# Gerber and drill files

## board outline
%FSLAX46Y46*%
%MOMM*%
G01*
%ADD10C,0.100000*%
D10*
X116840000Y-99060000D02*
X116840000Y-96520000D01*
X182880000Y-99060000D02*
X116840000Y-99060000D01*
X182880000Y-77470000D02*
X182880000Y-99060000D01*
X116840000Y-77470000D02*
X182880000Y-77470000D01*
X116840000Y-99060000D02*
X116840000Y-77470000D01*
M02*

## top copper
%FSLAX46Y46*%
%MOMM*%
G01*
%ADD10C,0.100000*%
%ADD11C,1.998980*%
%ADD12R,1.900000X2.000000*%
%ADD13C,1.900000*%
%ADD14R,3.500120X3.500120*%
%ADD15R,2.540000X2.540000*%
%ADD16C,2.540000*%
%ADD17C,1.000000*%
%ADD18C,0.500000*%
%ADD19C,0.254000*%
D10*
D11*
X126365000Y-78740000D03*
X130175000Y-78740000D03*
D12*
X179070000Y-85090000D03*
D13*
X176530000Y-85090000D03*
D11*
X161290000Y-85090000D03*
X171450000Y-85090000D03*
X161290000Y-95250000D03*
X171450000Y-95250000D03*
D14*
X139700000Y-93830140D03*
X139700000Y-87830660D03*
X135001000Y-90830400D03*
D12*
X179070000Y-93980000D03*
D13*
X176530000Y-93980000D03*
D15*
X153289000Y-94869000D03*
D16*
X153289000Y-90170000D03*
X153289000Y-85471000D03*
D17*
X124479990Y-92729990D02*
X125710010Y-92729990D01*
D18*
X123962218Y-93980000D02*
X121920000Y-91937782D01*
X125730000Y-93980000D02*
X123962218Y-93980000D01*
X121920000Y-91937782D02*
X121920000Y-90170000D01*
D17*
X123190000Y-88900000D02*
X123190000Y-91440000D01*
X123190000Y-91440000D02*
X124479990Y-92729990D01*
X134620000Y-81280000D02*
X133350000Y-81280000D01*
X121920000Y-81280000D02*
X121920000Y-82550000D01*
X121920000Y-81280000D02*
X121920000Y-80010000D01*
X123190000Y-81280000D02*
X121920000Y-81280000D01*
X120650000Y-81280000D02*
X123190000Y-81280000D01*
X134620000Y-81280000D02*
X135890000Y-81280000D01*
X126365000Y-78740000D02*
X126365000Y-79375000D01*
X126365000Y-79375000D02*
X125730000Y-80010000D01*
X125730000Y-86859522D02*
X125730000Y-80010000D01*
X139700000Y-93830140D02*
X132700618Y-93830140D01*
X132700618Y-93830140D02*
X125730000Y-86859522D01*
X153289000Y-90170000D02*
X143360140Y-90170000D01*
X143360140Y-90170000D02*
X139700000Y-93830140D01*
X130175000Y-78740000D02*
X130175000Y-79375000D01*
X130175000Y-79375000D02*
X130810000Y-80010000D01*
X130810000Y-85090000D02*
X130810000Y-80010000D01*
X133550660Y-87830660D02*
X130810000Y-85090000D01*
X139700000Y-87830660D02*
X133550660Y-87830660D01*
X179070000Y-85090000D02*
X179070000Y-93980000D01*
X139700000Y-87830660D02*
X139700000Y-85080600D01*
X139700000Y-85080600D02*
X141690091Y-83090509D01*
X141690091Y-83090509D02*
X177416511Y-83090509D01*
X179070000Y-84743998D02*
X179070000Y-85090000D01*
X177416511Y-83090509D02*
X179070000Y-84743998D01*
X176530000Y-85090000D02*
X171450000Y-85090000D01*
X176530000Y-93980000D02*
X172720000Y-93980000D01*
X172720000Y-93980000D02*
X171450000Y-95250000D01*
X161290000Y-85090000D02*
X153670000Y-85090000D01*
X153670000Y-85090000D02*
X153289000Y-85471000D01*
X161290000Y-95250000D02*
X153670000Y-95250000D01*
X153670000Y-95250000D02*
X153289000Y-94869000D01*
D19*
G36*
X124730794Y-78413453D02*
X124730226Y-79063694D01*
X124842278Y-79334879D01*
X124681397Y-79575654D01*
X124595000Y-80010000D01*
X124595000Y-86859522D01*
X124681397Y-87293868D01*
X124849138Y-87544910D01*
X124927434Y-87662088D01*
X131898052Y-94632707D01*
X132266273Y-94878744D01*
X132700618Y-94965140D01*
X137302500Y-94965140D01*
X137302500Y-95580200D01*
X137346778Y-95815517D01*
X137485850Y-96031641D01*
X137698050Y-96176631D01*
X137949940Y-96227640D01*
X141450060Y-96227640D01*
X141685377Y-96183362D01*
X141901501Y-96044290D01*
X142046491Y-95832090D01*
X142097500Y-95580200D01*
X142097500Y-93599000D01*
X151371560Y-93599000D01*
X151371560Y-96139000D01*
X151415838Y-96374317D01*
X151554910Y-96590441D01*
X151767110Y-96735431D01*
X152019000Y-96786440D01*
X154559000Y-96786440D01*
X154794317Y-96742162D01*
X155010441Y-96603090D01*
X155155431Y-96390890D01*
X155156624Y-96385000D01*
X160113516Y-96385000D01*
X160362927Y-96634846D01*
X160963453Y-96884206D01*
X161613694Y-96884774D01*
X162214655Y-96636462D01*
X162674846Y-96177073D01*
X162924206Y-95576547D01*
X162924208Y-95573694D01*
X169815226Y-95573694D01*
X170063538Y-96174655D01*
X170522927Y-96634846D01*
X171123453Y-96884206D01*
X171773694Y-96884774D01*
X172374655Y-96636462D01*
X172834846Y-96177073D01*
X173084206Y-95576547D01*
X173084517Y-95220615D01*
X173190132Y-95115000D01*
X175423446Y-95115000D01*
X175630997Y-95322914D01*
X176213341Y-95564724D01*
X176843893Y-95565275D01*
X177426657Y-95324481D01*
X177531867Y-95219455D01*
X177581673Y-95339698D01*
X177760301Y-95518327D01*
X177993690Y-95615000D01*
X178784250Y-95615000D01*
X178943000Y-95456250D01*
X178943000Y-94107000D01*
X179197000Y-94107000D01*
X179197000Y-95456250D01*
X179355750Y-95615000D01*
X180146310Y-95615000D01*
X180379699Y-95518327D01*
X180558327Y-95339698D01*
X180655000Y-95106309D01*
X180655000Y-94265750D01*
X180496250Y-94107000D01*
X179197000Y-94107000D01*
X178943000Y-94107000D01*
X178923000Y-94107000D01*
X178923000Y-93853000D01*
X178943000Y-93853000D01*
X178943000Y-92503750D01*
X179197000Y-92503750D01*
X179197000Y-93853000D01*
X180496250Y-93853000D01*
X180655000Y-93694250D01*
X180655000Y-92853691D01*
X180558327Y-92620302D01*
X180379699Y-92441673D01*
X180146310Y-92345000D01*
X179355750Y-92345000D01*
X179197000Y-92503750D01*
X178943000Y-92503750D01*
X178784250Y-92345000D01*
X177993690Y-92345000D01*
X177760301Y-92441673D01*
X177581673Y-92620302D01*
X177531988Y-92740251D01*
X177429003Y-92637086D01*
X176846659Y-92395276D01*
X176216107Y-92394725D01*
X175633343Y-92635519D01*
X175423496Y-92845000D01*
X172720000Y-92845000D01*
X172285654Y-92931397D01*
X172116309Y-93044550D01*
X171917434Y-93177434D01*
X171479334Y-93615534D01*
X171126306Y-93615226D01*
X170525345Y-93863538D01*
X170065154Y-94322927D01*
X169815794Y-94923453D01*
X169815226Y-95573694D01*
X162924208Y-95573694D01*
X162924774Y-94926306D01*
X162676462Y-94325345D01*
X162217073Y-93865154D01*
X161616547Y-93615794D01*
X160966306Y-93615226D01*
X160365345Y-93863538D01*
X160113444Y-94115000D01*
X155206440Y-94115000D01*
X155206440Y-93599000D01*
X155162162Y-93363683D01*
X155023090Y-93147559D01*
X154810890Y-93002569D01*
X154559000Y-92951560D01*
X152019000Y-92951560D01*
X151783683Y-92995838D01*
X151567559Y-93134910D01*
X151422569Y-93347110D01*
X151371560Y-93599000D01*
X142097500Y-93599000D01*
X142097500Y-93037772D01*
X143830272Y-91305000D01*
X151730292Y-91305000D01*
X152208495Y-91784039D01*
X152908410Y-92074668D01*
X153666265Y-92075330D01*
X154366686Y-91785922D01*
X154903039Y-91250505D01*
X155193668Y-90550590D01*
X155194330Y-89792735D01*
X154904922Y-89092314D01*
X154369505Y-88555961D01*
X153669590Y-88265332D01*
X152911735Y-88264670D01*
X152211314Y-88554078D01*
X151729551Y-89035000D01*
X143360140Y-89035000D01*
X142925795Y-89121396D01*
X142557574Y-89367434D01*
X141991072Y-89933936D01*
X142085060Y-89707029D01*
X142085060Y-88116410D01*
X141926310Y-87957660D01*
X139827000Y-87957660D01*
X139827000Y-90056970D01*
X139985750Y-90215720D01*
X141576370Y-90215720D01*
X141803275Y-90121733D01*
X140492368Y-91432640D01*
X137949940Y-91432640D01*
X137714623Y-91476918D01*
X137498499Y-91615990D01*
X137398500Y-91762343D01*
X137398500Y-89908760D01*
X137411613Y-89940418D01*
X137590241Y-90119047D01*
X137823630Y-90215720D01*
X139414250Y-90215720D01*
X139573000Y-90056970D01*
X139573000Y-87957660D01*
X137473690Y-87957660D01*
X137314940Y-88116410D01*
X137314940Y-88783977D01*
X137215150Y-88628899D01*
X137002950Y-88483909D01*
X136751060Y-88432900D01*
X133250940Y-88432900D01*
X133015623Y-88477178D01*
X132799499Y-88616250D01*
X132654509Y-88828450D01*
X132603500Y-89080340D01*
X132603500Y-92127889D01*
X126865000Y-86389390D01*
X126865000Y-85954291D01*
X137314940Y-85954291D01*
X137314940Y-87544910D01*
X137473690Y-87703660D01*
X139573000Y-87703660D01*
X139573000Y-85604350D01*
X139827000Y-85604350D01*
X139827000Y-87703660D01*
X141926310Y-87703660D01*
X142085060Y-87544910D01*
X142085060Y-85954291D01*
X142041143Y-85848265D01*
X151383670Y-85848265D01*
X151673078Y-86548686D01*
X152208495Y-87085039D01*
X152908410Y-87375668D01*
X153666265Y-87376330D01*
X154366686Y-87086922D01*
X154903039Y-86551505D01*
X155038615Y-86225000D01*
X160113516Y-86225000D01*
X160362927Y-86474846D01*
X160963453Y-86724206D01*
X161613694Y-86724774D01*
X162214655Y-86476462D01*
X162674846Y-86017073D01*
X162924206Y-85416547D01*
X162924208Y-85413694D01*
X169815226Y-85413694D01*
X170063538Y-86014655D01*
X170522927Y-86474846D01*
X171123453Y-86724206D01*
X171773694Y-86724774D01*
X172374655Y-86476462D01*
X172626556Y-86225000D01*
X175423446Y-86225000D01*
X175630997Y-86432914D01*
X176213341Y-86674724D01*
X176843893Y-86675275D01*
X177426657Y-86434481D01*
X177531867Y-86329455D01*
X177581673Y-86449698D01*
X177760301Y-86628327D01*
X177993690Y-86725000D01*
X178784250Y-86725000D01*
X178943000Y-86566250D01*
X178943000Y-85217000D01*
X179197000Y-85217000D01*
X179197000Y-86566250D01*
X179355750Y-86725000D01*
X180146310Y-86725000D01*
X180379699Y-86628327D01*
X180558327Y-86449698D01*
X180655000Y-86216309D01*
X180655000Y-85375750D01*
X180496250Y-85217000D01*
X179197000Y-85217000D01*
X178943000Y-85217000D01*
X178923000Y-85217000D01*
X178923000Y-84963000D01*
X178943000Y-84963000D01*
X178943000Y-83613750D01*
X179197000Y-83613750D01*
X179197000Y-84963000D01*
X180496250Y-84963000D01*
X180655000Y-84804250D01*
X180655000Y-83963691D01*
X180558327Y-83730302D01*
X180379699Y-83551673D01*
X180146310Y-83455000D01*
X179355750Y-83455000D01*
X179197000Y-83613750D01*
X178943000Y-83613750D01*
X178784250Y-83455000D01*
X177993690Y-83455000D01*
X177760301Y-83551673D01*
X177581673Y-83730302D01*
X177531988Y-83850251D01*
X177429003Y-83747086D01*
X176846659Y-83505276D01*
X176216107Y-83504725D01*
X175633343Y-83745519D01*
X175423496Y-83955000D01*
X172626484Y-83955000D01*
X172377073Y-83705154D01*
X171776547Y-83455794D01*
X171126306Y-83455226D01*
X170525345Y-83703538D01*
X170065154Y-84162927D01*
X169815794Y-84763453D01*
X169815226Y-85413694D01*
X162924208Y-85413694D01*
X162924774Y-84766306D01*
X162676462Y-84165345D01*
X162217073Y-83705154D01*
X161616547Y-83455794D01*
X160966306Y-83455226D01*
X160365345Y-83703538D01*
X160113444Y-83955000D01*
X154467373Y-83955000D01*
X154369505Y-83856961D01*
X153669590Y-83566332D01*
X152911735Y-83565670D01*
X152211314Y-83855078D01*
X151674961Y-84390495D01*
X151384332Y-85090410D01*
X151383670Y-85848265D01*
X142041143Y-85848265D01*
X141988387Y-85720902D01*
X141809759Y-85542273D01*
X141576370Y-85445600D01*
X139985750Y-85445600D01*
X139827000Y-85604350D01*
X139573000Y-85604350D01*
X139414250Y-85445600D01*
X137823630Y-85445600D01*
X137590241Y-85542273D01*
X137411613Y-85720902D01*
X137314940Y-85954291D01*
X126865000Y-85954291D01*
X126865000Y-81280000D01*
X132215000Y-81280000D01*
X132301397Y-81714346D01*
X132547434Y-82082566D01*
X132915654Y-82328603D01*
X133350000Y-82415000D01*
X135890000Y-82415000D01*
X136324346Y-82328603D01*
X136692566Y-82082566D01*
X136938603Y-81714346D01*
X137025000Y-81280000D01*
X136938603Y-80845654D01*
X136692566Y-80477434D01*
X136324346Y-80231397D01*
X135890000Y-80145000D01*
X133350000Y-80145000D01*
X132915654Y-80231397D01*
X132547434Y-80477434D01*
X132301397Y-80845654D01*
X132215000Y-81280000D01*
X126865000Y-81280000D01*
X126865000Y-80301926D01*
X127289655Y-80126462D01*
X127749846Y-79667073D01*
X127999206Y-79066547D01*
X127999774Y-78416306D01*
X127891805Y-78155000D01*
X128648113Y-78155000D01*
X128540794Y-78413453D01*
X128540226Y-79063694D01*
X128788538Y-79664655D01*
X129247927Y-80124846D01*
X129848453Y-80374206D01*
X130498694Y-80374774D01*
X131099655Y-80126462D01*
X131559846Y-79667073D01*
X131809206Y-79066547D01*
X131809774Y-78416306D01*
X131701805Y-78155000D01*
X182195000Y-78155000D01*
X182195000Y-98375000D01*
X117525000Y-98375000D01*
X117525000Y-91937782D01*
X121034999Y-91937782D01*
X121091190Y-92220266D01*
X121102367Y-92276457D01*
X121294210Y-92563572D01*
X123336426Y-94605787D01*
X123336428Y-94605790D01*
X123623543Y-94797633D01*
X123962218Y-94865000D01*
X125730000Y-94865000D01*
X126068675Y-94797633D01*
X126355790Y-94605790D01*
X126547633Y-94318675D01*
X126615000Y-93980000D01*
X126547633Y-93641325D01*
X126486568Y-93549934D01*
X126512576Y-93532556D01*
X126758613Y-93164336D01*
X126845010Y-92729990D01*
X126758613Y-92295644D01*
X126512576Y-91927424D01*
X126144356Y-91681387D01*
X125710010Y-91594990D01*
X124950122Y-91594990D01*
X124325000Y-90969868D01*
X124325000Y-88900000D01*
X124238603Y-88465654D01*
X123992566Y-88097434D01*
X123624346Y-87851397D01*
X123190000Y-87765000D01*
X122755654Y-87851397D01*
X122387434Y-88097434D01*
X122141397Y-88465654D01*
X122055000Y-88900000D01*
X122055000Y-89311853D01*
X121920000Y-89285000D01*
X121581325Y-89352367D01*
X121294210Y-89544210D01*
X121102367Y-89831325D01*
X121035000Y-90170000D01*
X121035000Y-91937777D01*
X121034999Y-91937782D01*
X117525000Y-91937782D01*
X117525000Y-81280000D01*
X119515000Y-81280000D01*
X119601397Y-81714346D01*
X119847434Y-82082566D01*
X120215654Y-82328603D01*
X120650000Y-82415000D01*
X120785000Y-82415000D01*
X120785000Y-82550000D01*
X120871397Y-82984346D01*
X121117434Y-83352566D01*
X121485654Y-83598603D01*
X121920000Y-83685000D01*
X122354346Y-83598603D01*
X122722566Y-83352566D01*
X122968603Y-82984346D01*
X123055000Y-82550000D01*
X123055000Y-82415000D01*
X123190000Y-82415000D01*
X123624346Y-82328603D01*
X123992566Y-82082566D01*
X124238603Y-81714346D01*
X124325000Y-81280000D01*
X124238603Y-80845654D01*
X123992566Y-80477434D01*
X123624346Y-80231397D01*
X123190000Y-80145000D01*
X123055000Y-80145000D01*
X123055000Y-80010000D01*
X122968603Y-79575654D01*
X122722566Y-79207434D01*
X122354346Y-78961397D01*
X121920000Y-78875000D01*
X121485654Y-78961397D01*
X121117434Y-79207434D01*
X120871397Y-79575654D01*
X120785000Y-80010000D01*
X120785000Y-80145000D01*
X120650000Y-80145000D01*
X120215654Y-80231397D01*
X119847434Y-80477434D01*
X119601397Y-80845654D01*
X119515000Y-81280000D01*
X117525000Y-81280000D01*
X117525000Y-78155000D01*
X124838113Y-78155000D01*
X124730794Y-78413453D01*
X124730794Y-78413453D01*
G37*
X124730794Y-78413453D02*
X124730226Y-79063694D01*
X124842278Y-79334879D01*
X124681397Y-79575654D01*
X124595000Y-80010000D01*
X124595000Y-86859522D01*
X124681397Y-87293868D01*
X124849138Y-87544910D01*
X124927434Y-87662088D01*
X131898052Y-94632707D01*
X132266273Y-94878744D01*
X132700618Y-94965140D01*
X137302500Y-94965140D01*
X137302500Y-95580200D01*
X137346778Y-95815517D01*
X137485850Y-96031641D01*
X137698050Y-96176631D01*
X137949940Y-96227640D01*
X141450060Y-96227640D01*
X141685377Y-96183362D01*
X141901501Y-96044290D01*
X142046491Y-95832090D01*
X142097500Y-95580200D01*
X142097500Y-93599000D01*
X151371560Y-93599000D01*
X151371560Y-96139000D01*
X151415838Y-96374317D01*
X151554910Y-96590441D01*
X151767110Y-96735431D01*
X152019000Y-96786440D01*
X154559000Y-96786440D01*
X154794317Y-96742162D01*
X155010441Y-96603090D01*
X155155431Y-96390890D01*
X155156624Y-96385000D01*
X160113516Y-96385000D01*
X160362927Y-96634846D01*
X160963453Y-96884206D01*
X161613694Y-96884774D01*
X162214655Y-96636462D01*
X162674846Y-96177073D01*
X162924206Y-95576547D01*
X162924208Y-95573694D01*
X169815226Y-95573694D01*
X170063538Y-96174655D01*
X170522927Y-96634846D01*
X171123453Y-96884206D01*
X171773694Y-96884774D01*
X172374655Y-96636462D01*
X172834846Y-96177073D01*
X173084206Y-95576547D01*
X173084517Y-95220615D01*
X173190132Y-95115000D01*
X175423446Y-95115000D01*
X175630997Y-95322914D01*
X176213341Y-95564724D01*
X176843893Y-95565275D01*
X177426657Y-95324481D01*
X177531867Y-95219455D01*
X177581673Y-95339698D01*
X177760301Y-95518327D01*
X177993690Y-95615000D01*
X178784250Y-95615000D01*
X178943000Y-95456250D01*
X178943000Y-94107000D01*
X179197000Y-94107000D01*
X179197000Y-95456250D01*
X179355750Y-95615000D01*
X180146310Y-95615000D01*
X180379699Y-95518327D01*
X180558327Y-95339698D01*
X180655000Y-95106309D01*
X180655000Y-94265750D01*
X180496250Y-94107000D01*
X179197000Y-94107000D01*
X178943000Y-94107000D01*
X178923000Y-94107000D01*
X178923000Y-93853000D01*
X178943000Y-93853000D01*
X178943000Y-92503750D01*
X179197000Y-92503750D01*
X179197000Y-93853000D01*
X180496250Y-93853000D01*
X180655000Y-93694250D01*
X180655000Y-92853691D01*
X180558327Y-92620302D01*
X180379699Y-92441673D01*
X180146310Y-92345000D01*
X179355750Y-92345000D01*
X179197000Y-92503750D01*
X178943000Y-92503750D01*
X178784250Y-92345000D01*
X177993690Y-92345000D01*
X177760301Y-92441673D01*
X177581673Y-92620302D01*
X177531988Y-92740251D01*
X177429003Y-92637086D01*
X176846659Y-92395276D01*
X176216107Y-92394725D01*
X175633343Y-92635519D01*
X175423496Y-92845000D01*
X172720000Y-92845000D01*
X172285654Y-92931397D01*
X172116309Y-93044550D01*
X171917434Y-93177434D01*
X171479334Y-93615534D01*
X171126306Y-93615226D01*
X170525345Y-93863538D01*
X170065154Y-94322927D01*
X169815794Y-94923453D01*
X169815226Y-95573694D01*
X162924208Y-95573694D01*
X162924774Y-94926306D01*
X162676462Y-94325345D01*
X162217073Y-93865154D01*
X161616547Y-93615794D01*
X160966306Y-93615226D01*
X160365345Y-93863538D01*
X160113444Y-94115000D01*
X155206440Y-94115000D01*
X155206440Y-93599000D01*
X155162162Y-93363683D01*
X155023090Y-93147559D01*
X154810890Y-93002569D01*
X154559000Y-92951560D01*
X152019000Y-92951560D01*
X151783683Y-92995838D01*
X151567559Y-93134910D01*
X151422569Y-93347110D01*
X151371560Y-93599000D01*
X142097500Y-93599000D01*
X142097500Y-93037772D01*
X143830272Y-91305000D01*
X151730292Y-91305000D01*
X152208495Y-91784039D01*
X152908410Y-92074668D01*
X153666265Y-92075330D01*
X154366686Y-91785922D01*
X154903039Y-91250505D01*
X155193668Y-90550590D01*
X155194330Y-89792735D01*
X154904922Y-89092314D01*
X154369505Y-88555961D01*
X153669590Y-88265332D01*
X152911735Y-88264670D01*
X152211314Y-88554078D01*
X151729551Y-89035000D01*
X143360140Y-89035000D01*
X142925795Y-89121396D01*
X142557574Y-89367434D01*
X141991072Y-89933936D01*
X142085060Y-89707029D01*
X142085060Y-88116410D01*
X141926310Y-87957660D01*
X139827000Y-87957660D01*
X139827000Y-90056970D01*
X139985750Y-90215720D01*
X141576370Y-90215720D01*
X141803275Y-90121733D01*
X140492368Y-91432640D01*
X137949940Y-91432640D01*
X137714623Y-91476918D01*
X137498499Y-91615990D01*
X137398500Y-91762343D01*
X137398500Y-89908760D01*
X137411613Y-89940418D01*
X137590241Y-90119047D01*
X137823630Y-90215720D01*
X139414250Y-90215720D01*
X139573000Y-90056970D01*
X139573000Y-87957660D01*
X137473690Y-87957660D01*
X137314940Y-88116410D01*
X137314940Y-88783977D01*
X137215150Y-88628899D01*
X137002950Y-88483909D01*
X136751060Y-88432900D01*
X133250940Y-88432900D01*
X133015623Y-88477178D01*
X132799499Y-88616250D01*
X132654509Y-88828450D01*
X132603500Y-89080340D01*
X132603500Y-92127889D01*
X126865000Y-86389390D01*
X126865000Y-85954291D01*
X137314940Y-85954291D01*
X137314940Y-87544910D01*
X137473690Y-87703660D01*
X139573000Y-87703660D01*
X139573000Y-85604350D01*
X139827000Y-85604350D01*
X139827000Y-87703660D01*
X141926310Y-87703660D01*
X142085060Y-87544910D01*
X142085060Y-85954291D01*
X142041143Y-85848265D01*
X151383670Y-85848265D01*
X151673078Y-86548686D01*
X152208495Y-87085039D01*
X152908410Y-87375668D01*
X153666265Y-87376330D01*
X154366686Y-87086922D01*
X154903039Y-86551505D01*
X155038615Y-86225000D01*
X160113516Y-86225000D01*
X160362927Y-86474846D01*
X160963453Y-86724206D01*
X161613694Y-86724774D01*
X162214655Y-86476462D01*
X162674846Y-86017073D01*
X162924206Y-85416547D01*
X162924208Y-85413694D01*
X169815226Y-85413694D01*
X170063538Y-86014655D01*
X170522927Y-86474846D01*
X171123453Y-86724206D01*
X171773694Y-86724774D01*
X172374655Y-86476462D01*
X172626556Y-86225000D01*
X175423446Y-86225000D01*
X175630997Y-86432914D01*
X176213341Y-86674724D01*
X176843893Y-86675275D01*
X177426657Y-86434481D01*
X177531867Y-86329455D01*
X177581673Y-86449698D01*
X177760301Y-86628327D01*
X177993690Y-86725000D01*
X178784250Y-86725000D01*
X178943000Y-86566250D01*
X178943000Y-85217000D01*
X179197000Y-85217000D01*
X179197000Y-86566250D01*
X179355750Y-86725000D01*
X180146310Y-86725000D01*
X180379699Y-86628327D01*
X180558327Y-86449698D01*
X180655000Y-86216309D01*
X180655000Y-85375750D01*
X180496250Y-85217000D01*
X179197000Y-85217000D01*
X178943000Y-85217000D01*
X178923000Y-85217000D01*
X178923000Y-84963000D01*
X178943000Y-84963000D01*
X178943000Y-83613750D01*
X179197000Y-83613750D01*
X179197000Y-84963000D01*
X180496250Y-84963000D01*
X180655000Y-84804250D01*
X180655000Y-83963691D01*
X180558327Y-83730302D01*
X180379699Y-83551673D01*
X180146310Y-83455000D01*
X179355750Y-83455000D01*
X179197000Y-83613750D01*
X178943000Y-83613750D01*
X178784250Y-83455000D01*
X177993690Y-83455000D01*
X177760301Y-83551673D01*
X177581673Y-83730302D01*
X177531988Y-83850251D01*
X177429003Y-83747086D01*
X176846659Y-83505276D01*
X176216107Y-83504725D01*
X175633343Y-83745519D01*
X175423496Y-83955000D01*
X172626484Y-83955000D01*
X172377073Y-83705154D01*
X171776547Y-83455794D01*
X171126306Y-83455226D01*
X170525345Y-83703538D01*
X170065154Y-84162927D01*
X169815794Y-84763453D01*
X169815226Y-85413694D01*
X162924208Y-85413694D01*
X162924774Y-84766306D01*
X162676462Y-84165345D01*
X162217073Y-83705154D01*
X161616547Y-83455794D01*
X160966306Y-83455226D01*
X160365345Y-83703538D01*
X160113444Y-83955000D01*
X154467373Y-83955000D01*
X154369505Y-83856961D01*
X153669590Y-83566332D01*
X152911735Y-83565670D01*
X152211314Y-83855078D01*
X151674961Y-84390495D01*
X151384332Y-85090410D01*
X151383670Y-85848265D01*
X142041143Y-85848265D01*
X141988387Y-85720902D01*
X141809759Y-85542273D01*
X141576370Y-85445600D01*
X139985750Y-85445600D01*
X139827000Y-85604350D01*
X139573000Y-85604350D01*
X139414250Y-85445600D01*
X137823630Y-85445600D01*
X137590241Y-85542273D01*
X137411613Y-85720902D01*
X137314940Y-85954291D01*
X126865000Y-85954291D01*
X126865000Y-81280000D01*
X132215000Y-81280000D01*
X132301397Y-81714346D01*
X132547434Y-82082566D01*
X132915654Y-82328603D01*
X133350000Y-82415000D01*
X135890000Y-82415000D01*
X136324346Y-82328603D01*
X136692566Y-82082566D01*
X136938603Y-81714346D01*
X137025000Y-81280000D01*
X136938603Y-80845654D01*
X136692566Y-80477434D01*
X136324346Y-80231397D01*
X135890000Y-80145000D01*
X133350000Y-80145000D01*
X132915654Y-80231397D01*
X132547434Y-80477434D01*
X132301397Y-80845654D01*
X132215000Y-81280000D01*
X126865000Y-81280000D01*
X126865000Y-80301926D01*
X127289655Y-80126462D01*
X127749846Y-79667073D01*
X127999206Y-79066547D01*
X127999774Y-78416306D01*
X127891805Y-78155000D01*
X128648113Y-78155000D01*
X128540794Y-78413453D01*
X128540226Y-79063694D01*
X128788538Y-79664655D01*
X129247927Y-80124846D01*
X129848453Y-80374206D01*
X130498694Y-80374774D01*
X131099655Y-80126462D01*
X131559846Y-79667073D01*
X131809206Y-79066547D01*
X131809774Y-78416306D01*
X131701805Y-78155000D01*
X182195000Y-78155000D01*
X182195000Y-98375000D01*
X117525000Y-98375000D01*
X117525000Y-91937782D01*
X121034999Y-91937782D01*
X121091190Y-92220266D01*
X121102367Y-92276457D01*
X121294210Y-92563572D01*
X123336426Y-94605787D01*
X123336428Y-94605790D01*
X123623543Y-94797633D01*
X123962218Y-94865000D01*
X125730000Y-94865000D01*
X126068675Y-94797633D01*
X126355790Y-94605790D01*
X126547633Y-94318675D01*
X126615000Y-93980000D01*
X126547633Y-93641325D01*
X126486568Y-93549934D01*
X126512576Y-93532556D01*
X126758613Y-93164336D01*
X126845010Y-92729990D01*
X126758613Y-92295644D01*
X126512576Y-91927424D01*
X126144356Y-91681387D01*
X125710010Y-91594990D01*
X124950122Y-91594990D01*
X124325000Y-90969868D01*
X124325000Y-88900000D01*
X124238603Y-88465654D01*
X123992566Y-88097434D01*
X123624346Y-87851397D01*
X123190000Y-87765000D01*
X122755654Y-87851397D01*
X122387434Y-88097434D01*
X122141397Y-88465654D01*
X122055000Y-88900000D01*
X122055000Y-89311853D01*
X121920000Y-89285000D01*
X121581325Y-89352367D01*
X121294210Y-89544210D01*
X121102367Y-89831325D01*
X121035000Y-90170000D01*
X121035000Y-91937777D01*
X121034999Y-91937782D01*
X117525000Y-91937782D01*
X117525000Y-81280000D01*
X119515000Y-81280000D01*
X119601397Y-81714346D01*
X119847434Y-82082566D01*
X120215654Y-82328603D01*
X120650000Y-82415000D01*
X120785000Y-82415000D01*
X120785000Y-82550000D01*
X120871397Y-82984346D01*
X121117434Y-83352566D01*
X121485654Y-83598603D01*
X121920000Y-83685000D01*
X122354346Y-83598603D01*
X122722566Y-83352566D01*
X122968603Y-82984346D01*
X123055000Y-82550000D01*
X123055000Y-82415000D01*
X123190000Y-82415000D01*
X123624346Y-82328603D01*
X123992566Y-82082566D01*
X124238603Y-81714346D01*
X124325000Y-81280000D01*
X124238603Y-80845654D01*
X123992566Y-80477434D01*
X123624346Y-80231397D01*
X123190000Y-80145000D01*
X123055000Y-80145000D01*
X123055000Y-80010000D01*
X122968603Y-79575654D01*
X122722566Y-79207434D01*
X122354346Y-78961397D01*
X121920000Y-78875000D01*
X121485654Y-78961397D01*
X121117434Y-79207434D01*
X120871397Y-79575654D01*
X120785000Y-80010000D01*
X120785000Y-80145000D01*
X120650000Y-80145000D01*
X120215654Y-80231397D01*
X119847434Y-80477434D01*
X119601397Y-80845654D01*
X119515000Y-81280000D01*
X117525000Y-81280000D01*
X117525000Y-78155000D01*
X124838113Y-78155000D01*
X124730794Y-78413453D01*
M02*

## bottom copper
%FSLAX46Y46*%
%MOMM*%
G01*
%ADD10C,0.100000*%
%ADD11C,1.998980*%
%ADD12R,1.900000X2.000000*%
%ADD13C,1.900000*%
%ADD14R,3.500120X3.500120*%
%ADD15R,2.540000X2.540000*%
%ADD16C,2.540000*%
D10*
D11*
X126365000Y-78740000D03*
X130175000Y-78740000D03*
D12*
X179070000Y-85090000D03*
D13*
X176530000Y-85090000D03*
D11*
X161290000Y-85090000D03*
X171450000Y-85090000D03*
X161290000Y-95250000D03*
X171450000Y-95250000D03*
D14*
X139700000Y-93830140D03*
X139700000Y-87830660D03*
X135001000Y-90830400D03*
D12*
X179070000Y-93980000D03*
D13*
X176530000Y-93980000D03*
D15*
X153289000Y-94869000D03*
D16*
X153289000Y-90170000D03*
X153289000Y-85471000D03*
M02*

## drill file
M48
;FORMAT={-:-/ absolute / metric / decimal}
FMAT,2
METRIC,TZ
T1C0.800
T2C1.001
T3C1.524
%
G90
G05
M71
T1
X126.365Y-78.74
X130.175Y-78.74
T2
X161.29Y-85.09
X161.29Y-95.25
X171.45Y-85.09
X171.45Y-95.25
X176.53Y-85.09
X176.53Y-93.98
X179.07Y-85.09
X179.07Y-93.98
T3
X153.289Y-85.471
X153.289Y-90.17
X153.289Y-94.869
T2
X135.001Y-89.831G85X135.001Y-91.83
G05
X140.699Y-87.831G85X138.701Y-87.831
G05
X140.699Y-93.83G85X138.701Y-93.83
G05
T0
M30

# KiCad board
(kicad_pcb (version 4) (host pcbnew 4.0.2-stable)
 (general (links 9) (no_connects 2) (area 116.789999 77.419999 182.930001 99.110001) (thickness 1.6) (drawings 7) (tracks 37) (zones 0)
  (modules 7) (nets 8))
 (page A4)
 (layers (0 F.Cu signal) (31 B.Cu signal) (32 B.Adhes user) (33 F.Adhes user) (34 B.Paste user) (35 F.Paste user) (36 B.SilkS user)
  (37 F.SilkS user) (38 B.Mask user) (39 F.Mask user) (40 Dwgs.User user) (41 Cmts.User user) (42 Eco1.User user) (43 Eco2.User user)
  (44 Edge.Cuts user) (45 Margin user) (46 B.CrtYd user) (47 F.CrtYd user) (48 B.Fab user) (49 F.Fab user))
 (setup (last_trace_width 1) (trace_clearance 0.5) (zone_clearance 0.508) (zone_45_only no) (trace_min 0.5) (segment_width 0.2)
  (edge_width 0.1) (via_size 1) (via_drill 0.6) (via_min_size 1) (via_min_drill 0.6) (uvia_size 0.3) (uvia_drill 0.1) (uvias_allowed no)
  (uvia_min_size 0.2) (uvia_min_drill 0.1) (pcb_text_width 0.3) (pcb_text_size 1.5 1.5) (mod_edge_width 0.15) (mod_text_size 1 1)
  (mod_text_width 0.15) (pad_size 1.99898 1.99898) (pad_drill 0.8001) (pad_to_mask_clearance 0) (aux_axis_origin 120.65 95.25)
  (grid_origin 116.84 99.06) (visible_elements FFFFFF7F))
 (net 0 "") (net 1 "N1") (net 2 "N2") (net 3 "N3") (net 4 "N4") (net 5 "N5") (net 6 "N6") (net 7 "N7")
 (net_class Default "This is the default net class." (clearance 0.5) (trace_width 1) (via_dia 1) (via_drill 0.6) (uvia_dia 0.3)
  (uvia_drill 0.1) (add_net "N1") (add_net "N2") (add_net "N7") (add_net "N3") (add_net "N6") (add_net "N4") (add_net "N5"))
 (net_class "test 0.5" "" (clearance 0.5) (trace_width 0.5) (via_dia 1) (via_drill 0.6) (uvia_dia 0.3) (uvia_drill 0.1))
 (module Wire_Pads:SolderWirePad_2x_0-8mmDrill (layer F.Cu) (at 128.27 78.74)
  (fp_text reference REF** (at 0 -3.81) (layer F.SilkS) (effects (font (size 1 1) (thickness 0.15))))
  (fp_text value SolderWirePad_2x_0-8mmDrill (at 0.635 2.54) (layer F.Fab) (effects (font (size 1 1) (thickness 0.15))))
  (pad 1 thru_hole circle (at -1.905 0) (size 1.99898 1.99898) (drill 0.8001) (layers *.Cu *.Mask F.SilkS) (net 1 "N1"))
  (pad 1 thru_hole circle (at 1.905 0) (size 1.99898 1.99898) (drill 0.8001) (layers *.Cu *.Mask F.SilkS) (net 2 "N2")))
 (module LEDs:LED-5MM (layer F.Cu) (at 179.07 85.09 180)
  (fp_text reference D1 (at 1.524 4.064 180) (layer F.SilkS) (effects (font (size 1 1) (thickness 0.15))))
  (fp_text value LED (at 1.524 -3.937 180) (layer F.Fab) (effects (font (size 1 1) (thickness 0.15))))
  (pad 1 thru_hole rect (at 0 0 270) (size 2 1.9) (drill 1.00076) (layers *.Cu *.Mask F.SilkS) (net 2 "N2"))
  (pad 2 thru_hole circle (at 2.54 0 180) (size 1.9 1.9) (drill 1.00076) (layers *.Cu *.Mask F.SilkS) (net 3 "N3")))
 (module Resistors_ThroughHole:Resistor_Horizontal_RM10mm (layer F.Cu) (at 161.29 85.09)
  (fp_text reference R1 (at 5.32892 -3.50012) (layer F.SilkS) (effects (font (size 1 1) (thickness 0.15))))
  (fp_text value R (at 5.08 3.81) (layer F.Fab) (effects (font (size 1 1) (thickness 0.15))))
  (pad 1 thru_hole circle (at 0 0) (size 1.99898 1.99898) (drill 1.00076) (layers *.Cu *.SilkS *.Mask) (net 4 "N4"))
  (pad 2 thru_hole circle (at 10.16 0) (size 1.99898 1.99898) (drill 1.00076) (layers *.Cu *.SilkS *.Mask) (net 3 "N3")))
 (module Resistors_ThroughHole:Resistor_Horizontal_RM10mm (layer F.Cu) (at 161.29 95.25)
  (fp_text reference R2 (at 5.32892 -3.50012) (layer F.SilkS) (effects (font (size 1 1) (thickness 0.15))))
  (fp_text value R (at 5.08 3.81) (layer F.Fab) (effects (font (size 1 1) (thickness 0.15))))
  (pad 1 thru_hole circle (at 0 0) (size 1.99898 1.99898) (drill 1.00076) (layers *.Cu *.SilkS *.Mask) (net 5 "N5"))
  (pad 2 thru_hole circle (at 10.16 0) (size 1.99898 1.99898) (drill 1.00076) (layers *.Cu *.SilkS *.Mask) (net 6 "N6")))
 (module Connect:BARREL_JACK (layer F.Cu) (at 139.7 87.63 270)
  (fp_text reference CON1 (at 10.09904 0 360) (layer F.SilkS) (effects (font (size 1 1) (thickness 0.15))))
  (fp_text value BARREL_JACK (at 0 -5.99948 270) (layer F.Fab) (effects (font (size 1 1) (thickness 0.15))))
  (pad 1 thru_hole rect (at 6.20014 0 270) (size 3.50012 3.50012) (drill oval 1.00076 2.99974) (layers *.Cu *.Mask F.SilkS) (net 1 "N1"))
  (pad 2 thru_hole rect (at 0.20066 0 270) (size 3.50012 3.50012) (drill oval 1.00076 2.99974) (layers *.Cu *.Mask F.SilkS) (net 2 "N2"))
  (pad 3 thru_hole rect (at 3.2004 4.699 270) (size 3.50012 3.50012) (drill oval 2.99974 1.00076) (layers *.Cu *.Mask F.SilkS) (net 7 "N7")))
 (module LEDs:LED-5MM (layer F.Cu) (at 179.07 93.98 180)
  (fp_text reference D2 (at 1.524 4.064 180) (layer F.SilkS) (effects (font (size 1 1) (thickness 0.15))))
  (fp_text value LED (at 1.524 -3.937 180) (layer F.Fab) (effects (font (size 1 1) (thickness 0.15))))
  (pad 1 thru_hole rect (at 0 0 270) (size 2 1.9) (drill 1.00076) (layers *.Cu *.Mask F.SilkS) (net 2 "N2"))
  (pad 2 thru_hole circle (at 2.54 0 180) (size 1.9 1.9) (drill 1.00076) (layers *.Cu *.Mask F.SilkS) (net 6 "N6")))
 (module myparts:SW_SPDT (layer F.Cu) (at 153.289 90.17 90)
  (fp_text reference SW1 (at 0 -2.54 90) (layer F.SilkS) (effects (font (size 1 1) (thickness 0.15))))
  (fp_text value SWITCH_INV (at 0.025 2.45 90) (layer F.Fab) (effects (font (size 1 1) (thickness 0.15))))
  (pad 1 thru_hole rect (at -4.699 0 90) (size 2.54 2.54) (drill 1.524) (layers *.Cu *.Mask F.SilkS) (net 5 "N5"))
  (pad 2 thru_hole circle (at 0 0 90) (size 2.54 2.54) (drill 1.524) (layers *.Cu *.Mask F.SilkS) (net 1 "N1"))
  (pad 3 thru_hole circle (at 4.699 0 90) (size 2.54 2.54) (drill 1.524) (layers *.Cu *.Mask F.SilkS) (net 4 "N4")))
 (gr_line (start 116.84 99.06) (end 116.84 96.52) (layer Edge.Cuts) (width 0.1))
 (gr_line (start 182.88 99.06) (end 116.84 99.06) (layer Edge.Cuts) (width 0.1))
 (gr_line (start 182.88 77.47) (end 182.88 99.06) (layer Edge.Cuts) (width 0.1))
 (gr_line (start 116.84 77.47) (end 182.88 77.47) (layer Edge.Cuts) (width 0.1))
 (gr_line (start 116.84 99.06) (end 116.84 77.47) (layer Edge.Cuts) (width 0.1))
 (segment (start 124.47999 92.72999) (end 125.71001 92.72999) (width 1) (layer F.Cu) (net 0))
 (segment (start 123.962218 93.98) (end 121.92 91.937782) (width 0.5) (layer F.Cu) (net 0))
 (segment (start 125.73 93.98) (end 123.962218 93.98) (width 0.5) (layer F.Cu) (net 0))
 (segment (start 121.92 91.937782) (end 121.92 90.17) (width 0.5) (layer F.Cu) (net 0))
 (segment (start 123.19 88.9) (end 123.19 91.44) (width 1) (layer F.Cu) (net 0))
 (segment (start 123.19 91.44) (end 124.47999 92.72999) (width 1) (layer F.Cu) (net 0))
 (segment (start 134.62 81.28) (end 133.35 81.28) (width 1) (layer F.Cu) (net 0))
 (segment (start 121.92 81.28) (end 121.92 82.55) (width 1) (layer F.Cu) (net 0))
 (segment (start 121.92 81.28) (end 121.92 80.01) (width 1) (layer F.Cu) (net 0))
 (segment (start 123.19 81.28) (end 121.92 81.28) (width 1) (layer F.Cu) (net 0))
 (segment (start 120.65 81.28) (end 123.19 81.28) (width 1) (layer F.Cu) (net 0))
 (segment (start 134.62 81.28) (end 135.89 81.28) (width 1) (layer F.Cu) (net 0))
 (segment (start 126.365 78.74) (end 126.365 79.375) (width 1) (layer F.Cu) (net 1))
 (segment (start 126.365 79.375) (end 125.73 80.01) (width 1) (layer F.Cu) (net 1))
 (segment (start 125.73 86.859522) (end 125.73 80.01) (width 1) (layer F.Cu) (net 1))
 (segment (start 139.7 93.83014) (end 132.700618 93.83014) (width 1) (layer F.Cu) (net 1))
 (segment (start 132.700618 93.83014) (end 125.73 86.859522) (width 1) (layer F.Cu) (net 1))
 (segment (start 153.289 90.17) (end 143.36014 90.17) (width 1) (layer F.Cu) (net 1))
 (segment (start 143.36014 90.17) (end 139.7 93.83014) (width 1) (layer F.Cu) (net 1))
 (segment (start 130.175 78.74) (end 130.175 79.375) (width 1) (layer F.Cu) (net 2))
 (segment (start 130.175 79.375) (end 130.81 80.01) (width 1) (layer F.Cu) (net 2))
 (segment (start 130.81 85.09) (end 130.81 80.01) (width 1) (layer F.Cu) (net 2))
 (segment (start 133.55066 87.83066) (end 130.81 85.09) (width 1) (layer F.Cu) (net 2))
 (segment (start 139.7 87.83066) (end 133.55066 87.83066) (width 1) (layer F.Cu) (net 2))
 (segment (start 179.07 85.09) (end 179.07 93.98) (width 1) (layer F.Cu) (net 2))
 (segment (start 139.7 87.83066) (end 139.7 85.0806) (width 1) (layer F.Cu) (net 2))
 (segment (start 139.7 85.0806) (end 141.690091 83.090509) (width 1) (layer F.Cu) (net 2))
 (segment (start 141.690091 83.090509) (end 177.416511 83.090509) (width 1) (layer F.Cu) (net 2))
 (segment (start 179.07 84.743998) (end 179.07 85.09) (width 1) (layer F.Cu) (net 2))
 (segment (start 177.416511 83.090509) (end 179.07 84.743998) (width 1) (layer F.Cu) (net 2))
 (segment (start 176.53 85.09) (end 171.45 85.09) (width 1) (layer F.Cu) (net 3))
 (segment (start 176.53 93.98) (end 172.72 93.98) (width 1) (layer F.Cu) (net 6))
 (segment (start 172.72 93.98) (end 171.45 95.25) (width 1) (layer F.Cu) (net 6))
 (segment (start 161.29 85.09) (end 153.67 85.09) (width 1) (layer F.Cu) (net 4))
 (segment (start 153.67 85.09) (end 153.289 85.471) (width 1) (layer F.Cu) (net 4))
 (segment (start 161.29 95.25) (end 153.67 95.25) (width 1) (layer F.Cu) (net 5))
 (segment (start 153.67 95.25) (end 153.289 94.869) (width 1) (layer F.Cu) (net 5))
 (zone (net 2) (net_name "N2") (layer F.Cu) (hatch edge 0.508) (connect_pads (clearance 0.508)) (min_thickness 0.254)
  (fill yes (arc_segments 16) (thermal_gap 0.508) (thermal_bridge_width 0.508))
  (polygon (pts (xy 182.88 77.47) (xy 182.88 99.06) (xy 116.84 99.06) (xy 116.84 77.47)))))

